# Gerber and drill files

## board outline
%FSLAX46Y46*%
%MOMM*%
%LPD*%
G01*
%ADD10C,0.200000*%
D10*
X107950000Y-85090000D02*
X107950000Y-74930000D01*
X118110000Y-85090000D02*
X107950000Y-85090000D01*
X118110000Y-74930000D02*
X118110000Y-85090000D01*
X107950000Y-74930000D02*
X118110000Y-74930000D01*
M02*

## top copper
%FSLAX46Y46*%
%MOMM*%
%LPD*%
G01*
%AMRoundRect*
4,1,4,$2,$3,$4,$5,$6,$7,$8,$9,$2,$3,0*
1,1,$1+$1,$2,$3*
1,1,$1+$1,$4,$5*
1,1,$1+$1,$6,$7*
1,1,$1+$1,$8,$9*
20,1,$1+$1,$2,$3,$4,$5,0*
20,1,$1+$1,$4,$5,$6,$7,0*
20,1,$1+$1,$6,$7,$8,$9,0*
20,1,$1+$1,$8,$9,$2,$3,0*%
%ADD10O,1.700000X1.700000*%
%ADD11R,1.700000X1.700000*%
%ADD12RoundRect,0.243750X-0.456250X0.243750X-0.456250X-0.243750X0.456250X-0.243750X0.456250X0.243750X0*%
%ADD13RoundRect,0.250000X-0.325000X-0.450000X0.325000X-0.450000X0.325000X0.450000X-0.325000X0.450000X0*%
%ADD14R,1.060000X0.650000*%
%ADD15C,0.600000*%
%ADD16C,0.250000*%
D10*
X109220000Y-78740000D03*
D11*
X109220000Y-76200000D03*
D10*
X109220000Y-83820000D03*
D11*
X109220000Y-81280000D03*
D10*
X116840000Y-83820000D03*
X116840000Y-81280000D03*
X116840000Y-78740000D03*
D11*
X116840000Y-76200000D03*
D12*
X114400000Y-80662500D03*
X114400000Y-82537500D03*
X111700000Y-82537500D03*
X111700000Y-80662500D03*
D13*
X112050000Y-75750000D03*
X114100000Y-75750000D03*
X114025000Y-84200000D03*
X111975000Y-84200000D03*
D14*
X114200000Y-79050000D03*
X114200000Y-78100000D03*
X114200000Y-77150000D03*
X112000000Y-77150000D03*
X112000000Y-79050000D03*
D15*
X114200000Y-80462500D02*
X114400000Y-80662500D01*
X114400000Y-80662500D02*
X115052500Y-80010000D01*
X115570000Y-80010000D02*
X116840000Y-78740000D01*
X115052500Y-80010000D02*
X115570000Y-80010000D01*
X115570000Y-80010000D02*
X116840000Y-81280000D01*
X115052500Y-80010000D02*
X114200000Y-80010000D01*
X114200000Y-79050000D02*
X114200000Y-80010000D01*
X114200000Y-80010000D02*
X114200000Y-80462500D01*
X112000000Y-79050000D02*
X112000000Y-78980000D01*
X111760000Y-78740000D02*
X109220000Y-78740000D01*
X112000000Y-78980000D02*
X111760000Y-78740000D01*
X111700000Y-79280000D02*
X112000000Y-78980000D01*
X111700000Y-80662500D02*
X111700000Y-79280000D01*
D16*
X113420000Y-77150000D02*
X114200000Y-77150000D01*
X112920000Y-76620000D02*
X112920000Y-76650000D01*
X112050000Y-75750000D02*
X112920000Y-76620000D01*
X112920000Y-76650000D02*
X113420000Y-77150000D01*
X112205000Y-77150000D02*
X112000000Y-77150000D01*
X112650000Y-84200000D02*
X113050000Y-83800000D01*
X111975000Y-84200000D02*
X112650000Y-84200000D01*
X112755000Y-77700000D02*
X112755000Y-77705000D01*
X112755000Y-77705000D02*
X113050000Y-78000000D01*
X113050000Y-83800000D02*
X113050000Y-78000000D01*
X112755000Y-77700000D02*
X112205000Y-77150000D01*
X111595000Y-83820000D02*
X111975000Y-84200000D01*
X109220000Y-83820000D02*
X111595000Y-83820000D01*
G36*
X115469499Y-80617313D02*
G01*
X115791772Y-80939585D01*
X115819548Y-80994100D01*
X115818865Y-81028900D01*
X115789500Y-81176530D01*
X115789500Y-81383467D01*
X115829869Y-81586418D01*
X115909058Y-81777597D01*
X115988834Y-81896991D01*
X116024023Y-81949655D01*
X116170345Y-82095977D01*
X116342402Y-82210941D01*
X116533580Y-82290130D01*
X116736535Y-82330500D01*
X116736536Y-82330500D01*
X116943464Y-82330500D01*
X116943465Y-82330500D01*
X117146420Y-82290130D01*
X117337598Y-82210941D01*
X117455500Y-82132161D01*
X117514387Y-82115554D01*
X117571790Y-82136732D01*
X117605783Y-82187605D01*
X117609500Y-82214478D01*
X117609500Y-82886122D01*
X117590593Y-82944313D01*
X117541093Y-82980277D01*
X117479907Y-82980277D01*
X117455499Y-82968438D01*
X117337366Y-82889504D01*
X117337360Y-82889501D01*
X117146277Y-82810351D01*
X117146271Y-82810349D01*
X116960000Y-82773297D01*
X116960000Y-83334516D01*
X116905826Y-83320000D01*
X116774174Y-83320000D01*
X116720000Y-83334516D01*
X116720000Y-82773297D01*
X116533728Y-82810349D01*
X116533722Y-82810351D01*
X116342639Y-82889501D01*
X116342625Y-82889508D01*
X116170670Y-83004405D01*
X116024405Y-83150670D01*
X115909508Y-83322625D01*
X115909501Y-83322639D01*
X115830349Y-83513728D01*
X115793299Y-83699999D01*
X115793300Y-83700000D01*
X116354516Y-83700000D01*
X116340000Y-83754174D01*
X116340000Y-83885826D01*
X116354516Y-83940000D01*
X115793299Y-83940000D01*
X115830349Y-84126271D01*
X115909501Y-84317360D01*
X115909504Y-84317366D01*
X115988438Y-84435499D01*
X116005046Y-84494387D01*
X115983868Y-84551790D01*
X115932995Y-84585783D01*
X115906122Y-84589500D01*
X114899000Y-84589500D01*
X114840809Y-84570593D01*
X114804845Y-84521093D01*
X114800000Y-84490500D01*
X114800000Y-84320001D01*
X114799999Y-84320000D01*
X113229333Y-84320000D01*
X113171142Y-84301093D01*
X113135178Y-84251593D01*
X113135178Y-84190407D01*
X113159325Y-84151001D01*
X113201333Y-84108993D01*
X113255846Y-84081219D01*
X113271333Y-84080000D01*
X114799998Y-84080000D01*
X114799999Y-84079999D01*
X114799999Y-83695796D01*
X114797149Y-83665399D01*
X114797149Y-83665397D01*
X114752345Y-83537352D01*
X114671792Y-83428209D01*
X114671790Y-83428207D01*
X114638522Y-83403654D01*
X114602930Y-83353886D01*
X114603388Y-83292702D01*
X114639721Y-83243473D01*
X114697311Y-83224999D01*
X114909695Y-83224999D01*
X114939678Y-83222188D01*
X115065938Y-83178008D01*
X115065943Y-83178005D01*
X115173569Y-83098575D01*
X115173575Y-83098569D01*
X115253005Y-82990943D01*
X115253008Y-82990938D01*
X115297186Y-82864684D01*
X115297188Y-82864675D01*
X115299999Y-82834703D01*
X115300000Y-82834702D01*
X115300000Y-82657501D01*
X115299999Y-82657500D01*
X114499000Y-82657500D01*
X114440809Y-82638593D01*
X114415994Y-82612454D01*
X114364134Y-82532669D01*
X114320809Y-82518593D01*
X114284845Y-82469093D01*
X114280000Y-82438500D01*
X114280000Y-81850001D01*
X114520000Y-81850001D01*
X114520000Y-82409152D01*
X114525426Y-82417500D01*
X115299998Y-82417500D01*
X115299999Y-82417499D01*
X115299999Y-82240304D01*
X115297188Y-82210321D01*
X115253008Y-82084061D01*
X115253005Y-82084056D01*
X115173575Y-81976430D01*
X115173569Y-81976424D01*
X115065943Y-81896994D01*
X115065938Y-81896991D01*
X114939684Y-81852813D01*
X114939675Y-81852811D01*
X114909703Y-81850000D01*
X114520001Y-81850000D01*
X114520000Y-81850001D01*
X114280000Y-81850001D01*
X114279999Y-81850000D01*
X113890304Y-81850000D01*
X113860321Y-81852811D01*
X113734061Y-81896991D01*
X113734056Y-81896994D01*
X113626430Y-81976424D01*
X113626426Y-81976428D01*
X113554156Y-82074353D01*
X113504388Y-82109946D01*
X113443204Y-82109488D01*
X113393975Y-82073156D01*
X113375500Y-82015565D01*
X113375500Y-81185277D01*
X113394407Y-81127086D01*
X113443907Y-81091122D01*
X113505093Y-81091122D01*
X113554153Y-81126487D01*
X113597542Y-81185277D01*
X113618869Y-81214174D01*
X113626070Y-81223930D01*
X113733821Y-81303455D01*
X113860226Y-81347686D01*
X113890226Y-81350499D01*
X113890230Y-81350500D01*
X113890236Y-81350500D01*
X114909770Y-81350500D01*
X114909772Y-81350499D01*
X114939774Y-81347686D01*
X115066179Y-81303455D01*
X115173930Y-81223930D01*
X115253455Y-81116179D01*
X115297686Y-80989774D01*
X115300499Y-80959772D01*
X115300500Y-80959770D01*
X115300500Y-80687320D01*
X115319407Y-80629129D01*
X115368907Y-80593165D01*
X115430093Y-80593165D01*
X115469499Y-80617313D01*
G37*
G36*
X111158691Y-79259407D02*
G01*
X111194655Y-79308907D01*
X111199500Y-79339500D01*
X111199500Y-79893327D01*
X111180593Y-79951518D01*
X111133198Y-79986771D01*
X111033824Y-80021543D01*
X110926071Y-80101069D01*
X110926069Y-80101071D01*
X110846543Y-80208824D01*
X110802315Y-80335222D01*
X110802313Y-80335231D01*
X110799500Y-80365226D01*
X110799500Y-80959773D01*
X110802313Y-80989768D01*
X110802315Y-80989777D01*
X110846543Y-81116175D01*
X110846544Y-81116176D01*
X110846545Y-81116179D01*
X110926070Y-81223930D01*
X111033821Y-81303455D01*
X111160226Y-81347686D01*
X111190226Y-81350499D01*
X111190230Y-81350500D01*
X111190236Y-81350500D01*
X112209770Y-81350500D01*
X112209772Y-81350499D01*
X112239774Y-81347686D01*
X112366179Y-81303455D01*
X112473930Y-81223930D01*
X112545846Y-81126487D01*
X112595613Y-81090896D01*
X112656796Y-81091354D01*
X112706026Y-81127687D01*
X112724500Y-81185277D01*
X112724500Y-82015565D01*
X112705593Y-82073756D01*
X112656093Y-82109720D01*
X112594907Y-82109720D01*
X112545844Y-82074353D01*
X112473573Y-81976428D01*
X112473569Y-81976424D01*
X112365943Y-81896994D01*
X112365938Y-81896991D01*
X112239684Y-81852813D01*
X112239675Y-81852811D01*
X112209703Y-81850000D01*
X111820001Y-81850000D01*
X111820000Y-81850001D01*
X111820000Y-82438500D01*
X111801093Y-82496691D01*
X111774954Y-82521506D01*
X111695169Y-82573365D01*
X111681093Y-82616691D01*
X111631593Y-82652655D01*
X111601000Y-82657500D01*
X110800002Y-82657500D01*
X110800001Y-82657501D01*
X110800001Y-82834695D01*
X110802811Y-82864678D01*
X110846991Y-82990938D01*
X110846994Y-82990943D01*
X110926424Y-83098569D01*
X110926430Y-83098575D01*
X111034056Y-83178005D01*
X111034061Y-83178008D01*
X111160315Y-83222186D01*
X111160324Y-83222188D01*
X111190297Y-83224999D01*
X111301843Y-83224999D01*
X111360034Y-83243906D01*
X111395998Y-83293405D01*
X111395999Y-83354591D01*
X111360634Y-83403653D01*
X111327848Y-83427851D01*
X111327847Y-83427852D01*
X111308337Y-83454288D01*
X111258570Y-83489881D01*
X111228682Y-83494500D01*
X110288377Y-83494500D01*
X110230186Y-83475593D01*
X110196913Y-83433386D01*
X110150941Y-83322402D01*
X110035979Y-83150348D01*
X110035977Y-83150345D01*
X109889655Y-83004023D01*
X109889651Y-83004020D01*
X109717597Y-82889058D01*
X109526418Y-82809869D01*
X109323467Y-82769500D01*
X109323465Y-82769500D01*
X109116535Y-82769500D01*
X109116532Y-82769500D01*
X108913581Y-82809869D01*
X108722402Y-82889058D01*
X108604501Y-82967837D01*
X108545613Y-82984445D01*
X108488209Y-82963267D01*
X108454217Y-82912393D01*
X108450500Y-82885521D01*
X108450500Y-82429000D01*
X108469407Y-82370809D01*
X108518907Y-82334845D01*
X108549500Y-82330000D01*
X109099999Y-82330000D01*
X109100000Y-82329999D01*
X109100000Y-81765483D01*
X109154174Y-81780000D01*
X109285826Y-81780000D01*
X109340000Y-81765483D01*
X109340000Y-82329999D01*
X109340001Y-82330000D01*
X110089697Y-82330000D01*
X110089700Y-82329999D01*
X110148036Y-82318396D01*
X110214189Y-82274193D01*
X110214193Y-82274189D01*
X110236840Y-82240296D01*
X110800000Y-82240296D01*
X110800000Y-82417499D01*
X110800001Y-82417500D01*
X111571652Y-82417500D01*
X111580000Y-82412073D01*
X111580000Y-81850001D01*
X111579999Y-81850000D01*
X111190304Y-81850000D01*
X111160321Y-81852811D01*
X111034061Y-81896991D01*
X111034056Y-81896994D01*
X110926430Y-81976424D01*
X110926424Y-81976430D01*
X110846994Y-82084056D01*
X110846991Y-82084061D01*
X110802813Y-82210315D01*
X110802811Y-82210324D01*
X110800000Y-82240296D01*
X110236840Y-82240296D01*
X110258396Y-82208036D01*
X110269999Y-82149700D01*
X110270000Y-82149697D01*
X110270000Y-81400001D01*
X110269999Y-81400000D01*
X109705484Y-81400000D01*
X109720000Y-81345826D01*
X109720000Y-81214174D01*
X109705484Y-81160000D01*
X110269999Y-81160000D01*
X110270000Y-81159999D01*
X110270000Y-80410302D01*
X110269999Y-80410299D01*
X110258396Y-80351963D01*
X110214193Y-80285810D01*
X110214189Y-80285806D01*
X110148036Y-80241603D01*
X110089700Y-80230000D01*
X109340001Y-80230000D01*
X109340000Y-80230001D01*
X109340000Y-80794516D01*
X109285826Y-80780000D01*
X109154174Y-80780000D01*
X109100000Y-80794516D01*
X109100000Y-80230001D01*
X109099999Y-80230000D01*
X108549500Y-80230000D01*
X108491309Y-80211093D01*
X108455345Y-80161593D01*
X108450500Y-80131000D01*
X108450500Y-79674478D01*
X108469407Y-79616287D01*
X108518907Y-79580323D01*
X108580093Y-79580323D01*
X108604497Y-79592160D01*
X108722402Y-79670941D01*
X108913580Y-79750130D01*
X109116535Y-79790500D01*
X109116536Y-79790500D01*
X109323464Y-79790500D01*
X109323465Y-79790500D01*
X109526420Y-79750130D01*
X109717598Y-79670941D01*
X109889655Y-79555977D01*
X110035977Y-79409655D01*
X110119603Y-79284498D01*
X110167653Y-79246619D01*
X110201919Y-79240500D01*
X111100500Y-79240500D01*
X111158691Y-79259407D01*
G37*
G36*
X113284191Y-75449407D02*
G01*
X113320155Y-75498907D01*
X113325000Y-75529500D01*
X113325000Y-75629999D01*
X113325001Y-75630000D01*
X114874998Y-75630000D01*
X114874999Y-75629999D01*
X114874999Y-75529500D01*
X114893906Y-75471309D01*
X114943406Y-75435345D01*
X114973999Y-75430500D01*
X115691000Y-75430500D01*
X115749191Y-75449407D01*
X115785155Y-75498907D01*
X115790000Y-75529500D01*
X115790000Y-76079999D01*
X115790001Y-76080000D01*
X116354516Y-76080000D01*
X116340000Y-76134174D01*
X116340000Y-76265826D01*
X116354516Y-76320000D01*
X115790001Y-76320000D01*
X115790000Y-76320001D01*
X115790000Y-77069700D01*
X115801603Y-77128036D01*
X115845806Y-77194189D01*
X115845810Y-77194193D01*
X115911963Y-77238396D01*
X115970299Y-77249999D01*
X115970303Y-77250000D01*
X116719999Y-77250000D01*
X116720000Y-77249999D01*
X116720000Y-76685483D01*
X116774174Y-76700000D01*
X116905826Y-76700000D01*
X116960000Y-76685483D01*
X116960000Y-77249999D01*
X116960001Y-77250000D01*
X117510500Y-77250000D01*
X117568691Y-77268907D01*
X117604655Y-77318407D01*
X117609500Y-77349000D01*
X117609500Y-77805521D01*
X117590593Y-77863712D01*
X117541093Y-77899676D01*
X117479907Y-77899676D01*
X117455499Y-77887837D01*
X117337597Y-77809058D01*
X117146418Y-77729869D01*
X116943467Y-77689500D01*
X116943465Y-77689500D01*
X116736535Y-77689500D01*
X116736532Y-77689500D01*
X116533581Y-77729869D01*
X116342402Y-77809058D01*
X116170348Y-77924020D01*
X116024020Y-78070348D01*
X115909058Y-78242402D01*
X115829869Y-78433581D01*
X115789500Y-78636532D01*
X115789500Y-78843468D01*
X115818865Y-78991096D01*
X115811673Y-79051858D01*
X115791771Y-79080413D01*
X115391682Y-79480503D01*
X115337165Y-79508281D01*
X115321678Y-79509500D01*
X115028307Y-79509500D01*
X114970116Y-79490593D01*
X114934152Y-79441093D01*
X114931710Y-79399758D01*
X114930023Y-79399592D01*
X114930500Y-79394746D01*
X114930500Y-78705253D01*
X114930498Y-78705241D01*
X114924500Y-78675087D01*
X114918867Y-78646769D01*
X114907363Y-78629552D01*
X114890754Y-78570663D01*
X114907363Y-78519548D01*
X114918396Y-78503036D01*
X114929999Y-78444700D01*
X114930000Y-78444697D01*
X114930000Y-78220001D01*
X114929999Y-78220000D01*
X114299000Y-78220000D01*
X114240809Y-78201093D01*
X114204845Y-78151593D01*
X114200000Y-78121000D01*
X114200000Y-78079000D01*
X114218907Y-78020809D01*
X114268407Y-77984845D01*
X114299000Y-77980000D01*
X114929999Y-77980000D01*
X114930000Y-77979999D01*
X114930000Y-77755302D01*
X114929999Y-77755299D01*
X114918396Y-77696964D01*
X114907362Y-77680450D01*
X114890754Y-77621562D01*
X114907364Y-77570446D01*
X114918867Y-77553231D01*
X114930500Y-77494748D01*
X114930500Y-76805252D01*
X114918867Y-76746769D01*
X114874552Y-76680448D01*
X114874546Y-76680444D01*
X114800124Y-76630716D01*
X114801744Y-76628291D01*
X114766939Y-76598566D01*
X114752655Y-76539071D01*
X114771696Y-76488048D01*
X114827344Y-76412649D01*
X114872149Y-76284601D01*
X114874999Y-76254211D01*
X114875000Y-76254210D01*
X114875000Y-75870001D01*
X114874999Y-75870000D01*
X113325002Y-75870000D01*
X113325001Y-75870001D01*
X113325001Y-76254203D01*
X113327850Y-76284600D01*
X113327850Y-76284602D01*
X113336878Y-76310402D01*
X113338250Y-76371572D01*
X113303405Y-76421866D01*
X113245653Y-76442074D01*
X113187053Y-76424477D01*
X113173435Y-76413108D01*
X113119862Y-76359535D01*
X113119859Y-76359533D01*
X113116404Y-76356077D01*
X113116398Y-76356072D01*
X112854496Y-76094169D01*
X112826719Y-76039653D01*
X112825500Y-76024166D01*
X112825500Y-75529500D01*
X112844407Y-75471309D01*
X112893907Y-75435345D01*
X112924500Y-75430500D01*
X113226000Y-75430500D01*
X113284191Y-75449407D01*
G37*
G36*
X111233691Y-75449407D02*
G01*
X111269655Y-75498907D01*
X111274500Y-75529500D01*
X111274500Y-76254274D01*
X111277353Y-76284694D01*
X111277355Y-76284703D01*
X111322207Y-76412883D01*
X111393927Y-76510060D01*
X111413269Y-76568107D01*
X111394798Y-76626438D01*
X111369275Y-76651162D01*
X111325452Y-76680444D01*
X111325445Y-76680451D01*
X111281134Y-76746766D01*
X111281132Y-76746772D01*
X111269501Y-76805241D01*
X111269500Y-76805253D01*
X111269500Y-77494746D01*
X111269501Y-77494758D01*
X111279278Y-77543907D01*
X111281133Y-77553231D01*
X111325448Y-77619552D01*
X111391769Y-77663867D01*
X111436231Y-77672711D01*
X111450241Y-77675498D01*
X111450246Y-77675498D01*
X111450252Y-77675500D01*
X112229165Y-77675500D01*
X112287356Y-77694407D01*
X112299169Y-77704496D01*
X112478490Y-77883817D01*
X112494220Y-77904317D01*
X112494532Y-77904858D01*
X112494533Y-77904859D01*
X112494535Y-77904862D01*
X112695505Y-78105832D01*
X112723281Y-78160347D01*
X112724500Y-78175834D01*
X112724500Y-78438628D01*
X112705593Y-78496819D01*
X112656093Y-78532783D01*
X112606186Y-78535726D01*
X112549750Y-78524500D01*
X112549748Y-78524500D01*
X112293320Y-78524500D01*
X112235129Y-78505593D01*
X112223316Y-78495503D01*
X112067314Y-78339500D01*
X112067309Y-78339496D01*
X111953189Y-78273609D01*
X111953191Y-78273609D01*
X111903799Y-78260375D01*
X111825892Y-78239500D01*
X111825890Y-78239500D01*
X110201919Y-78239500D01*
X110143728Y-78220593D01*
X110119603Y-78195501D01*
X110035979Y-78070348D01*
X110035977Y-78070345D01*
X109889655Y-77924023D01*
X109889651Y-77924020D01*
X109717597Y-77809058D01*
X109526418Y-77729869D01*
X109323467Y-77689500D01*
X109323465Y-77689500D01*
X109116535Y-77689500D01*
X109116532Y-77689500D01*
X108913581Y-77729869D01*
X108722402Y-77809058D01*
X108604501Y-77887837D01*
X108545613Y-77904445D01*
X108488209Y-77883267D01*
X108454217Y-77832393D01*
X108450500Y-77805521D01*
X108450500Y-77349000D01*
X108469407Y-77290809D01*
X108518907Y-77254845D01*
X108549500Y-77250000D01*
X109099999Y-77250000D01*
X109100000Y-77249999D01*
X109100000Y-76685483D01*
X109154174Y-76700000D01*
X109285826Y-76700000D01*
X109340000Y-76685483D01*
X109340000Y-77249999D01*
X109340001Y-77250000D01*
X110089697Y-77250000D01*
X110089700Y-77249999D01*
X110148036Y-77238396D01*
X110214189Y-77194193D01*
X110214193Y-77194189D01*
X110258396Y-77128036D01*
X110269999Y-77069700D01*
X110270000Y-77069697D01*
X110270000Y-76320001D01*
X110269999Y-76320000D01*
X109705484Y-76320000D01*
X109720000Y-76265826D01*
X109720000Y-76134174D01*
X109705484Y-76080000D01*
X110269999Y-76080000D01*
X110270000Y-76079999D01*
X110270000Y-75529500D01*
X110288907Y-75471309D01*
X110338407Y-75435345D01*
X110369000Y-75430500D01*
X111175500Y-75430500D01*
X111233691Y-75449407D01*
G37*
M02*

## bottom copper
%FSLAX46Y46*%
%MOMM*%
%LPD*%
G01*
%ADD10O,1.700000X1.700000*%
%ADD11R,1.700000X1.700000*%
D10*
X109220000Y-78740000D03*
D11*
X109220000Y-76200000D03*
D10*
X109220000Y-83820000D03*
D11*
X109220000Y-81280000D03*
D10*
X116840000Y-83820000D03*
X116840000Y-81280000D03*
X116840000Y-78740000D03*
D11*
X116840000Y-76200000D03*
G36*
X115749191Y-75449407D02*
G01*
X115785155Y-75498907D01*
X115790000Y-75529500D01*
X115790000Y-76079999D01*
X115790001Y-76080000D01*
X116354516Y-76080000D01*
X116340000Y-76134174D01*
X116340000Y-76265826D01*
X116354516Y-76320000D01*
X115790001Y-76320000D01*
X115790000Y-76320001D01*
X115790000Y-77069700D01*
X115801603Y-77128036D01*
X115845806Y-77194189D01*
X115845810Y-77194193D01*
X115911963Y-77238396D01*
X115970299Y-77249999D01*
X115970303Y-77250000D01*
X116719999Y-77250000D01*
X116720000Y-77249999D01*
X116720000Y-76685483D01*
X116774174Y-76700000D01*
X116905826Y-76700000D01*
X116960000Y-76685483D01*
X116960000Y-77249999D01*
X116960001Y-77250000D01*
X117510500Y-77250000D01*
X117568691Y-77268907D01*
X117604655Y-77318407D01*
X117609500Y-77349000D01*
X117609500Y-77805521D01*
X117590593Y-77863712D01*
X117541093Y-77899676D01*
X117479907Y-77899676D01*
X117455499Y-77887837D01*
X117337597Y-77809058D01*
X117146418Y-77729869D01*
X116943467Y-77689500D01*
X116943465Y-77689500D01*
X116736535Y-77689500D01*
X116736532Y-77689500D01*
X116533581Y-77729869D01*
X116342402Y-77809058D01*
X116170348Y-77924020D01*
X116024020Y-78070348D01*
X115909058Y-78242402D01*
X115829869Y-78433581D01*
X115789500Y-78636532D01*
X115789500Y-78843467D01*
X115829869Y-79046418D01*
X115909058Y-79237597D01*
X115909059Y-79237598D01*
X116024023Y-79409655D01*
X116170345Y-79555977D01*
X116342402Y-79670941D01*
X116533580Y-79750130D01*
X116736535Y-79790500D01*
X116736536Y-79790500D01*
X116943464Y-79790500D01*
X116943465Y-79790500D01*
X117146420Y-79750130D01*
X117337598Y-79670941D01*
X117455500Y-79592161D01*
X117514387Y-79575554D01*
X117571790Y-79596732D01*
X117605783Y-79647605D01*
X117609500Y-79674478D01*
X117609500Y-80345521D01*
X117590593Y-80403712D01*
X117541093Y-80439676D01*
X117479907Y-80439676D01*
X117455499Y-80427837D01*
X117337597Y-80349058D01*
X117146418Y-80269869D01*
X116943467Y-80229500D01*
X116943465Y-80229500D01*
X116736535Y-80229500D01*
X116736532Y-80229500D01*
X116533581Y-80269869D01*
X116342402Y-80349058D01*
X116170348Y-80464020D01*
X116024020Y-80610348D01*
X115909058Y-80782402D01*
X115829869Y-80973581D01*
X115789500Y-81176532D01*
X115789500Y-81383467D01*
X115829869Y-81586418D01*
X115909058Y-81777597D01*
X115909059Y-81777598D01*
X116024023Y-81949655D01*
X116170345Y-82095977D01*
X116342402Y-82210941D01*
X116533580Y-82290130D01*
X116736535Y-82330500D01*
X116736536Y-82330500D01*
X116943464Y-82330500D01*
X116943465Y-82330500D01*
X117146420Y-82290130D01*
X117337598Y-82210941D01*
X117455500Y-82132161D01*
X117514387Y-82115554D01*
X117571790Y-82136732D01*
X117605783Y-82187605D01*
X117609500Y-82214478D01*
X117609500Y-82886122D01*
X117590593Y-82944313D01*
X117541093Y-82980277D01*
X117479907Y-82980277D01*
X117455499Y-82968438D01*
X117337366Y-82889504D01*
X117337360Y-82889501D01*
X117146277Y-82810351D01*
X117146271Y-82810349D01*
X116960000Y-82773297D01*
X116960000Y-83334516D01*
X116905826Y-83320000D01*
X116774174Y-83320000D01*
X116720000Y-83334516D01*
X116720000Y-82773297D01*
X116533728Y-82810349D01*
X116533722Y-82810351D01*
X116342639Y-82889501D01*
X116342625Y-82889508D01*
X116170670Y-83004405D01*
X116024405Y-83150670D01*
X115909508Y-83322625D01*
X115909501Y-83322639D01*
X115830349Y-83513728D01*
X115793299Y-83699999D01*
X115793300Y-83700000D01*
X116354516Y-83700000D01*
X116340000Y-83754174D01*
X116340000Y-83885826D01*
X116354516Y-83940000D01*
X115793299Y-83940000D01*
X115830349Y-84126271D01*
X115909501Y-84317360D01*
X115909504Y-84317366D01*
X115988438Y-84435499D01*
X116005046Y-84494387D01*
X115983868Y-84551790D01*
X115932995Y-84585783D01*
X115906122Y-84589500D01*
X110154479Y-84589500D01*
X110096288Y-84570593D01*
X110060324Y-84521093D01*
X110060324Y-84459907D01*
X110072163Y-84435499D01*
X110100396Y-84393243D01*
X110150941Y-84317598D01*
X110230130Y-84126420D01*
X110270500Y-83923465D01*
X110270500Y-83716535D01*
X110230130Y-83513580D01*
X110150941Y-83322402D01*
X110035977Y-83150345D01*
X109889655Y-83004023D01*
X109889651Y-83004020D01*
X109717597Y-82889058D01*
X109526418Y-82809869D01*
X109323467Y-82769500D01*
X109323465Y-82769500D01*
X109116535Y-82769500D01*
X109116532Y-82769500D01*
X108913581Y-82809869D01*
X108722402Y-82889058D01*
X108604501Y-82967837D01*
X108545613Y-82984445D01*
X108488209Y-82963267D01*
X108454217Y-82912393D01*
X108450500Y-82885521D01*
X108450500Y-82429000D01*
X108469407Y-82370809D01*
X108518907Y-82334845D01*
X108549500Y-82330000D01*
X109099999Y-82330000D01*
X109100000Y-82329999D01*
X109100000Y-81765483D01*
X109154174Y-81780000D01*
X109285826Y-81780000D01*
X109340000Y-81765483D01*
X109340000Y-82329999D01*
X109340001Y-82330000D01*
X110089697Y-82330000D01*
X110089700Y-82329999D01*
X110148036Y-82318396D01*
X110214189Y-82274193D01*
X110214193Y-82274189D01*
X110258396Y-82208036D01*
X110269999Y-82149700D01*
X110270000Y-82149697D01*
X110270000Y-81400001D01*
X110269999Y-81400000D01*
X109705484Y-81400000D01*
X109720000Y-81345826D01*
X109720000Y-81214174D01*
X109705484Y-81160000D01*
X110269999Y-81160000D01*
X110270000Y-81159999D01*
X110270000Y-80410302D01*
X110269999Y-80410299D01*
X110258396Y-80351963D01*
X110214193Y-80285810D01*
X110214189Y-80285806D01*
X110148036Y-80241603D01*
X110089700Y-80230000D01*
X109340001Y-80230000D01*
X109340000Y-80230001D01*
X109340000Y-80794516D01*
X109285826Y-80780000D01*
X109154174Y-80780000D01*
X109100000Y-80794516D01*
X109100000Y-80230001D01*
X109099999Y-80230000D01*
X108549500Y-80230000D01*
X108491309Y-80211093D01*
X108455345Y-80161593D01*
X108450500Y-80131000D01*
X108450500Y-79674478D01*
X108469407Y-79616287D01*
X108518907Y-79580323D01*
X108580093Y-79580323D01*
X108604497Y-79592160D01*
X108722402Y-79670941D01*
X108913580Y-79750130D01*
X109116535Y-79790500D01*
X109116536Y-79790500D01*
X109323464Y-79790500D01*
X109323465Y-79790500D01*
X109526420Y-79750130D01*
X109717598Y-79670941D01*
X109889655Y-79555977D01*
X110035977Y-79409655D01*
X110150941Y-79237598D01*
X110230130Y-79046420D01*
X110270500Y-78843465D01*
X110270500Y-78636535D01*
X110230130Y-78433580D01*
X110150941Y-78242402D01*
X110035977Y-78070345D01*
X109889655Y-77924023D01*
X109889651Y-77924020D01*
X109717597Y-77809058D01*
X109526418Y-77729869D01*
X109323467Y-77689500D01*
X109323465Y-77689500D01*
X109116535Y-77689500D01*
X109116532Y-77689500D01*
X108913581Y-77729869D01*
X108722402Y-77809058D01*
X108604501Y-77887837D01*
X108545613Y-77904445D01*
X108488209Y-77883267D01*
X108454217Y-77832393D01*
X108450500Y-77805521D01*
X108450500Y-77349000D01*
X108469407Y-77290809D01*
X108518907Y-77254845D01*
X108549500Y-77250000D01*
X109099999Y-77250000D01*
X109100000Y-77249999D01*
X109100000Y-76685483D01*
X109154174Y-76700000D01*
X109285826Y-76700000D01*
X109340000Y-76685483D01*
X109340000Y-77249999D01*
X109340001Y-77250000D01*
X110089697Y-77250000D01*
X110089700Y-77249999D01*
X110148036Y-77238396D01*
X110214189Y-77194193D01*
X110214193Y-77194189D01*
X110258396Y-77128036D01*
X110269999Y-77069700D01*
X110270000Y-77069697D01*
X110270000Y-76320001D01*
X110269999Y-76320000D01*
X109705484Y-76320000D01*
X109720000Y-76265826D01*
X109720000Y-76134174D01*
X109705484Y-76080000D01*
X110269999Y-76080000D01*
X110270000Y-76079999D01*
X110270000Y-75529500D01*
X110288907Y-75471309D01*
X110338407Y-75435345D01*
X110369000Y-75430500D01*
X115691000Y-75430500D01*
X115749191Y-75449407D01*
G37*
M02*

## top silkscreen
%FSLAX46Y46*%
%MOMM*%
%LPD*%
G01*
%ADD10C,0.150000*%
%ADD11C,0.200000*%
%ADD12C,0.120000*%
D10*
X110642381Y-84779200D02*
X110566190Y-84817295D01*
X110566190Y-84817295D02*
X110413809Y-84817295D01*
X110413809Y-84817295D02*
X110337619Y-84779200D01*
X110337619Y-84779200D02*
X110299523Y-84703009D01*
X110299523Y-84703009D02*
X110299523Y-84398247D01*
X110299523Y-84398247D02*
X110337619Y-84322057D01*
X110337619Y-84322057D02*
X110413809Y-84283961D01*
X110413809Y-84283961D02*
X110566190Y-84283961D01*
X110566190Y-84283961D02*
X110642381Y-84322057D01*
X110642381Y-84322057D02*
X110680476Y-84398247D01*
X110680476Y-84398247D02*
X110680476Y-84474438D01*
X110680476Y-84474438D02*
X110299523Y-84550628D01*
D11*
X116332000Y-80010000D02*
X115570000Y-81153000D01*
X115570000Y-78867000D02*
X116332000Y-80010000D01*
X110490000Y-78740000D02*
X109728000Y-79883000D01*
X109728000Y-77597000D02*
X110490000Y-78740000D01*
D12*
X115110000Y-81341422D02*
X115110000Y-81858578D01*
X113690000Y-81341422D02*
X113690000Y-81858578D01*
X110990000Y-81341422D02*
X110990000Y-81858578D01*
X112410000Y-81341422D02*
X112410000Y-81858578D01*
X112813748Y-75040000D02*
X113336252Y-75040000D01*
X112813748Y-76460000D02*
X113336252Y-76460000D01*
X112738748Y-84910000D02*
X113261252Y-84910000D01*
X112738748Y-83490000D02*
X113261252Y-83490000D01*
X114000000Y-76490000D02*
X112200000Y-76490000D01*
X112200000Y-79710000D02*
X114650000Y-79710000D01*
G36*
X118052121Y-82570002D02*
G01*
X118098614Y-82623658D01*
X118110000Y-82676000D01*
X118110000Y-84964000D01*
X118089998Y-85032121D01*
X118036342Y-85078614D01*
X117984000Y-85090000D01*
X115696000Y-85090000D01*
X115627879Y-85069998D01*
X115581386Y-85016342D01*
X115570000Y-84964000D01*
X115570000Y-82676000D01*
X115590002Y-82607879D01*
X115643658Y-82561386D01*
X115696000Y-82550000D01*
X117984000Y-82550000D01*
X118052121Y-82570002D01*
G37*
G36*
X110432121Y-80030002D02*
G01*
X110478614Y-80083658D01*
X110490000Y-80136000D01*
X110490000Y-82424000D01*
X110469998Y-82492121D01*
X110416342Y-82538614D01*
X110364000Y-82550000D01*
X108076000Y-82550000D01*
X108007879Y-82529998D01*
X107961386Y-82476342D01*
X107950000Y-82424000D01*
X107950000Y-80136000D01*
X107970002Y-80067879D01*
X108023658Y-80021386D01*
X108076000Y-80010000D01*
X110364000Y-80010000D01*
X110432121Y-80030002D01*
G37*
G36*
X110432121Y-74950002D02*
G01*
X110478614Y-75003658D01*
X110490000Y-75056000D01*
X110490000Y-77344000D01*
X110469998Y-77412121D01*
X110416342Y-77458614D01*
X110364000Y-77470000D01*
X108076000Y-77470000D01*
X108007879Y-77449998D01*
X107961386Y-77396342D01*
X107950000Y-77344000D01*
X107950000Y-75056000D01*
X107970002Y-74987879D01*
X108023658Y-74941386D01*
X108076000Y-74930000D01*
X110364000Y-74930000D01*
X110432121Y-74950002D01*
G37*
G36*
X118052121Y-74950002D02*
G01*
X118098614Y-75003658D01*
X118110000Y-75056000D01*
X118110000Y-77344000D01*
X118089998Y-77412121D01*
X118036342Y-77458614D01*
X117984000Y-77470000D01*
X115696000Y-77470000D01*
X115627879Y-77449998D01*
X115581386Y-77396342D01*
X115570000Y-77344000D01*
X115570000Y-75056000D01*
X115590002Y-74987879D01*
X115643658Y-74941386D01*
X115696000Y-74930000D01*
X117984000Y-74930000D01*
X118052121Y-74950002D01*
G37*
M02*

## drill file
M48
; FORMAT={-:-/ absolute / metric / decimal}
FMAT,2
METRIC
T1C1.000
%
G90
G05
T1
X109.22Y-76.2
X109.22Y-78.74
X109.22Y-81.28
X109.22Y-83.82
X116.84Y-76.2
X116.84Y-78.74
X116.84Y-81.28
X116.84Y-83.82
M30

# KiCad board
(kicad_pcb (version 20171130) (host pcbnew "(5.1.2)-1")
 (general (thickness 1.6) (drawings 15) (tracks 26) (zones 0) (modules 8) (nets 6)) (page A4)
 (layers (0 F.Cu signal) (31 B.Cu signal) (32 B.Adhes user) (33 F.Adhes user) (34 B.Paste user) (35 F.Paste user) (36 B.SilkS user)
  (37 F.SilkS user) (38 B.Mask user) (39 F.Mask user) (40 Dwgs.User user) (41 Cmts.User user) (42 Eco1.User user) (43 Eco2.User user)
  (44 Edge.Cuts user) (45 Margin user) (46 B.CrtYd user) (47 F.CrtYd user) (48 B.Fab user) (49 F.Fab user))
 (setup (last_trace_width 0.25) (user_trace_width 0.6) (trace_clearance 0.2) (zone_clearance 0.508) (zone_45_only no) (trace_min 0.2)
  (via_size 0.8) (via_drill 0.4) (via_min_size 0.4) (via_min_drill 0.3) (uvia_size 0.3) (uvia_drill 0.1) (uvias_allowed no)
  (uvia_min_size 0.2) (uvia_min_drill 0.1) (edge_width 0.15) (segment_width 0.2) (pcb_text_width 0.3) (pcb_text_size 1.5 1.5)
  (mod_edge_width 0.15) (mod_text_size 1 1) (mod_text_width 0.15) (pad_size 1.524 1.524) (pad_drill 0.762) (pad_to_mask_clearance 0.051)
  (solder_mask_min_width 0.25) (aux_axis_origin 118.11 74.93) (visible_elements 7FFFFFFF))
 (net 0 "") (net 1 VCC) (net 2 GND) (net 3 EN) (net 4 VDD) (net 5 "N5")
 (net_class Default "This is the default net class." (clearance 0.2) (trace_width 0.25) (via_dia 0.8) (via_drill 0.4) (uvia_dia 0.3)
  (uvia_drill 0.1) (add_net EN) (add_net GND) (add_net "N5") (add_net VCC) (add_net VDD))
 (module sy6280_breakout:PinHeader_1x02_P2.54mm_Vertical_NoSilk (layer F.Cu) (at 109.22 76.2)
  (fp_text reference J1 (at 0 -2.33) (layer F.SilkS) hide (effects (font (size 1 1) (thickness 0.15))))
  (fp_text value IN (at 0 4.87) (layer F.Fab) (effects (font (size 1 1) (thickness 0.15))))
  (pad 2 thru_hole oval (at 0 2.54) (size 1.7 1.7) (drill 1) (layers *.Cu *.Mask) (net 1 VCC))
  (pad 1 thru_hole rect (at 0 0) (size 1.7 1.7) (drill 1) (layers *.Cu *.Mask) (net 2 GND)))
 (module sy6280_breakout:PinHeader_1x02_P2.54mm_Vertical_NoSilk (layer F.Cu) (at 109.22 81.28)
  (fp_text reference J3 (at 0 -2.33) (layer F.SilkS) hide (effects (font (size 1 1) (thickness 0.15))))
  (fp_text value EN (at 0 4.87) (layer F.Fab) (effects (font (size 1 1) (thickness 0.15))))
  (pad 2 thru_hole oval (at 0 2.54) (size 1.7 1.7) (drill 1) (layers *.Cu *.Mask) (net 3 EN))
  (pad 1 thru_hole rect (at 0 0) (size 1.7 1.7) (drill 1) (layers *.Cu *.Mask) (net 2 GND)))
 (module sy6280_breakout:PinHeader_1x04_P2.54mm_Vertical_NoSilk (layer F.Cu) (at 116.84 76.2)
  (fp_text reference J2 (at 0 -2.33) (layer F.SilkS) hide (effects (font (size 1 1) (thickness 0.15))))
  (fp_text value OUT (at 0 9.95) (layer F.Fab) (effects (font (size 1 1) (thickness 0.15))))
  (pad 4 thru_hole oval (at 0 7.62) (size 1.7 1.7) (drill 1) (layers *.Cu *.Mask) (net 2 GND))
  (pad 3 thru_hole oval (at 0 5.08) (size 1.7 1.7) (drill 1) (layers *.Cu *.Mask) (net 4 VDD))
  (pad 2 thru_hole oval (at 0 2.54) (size 1.7 1.7) (drill 1) (layers *.Cu *.Mask) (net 4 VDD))
  (pad 1 thru_hole rect (at 0 0) (size 1.7 1.7) (drill 1) (layers *.Cu *.Mask) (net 2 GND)))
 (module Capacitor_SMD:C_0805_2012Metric (layer F.Cu) (at 114.4 81.6 270)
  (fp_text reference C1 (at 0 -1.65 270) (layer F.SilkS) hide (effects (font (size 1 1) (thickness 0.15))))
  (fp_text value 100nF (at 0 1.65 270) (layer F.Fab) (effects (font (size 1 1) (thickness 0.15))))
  (fp_line (start -0.258578 -0.71) (end 0.258578 -0.71) (layer F.SilkS) (width 0.12))
  (fp_line (start -0.258578 0.71) (end 0.258578 0.71) (layer F.SilkS) (width 0.12))
  (pad 1 smd roundrect (at -0.9375 0 270) (size 0.975 1.4) (layers F.Cu F.Paste F.Mask) (roundrect_rratio 0.25) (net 4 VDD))
  (pad 2 smd roundrect (at 0.9375 0 270) (size 0.975 1.4) (layers F.Cu F.Paste F.Mask) (roundrect_rratio 0.25) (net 2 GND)))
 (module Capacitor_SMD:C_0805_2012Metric (layer F.Cu) (at 111.7 81.6 270)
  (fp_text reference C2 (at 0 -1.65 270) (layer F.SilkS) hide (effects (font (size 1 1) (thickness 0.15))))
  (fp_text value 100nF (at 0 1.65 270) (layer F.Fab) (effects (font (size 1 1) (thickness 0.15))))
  (fp_line (start -0.258578 0.71) (end 0.258578 0.71) (layer F.SilkS) (width 0.12))
  (fp_line (start -0.258578 -0.71) (end 0.258578 -0.71) (layer F.SilkS) (width 0.12))
  (pad 2 smd roundrect (at 0.9375 0 270) (size 0.975 1.4) (layers F.Cu F.Paste F.Mask) (roundrect_rratio 0.25) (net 2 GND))
  (pad 1 smd roundrect (at -0.9375 0 270) (size 0.975 1.4) (layers F.Cu F.Paste F.Mask) (roundrect_rratio 0.25) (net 1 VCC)))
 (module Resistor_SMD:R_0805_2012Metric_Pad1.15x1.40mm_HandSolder (layer F.Cu) (at 113.075 75.75)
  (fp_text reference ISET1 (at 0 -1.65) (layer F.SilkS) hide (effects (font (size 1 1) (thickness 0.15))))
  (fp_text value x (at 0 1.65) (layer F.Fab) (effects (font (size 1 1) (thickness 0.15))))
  (fp_line (start -0.261252 -0.71) (end 0.261252 -0.71) (layer F.SilkS) (width 0.12))
  (fp_line (start -0.261252 0.71) (end 0.261252 0.71) (layer F.SilkS) (width 0.12))
  (pad 1 smd roundrect (at -1.025 0) (size 1.15 1.4) (layers F.Cu F.Paste F.Mask) (roundrect_rratio 0.217391) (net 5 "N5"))
  (pad 2 smd roundrect (at 1.025 0) (size 1.15 1.4) (layers F.Cu F.Paste F.Mask) (roundrect_rratio 0.217391) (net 2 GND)))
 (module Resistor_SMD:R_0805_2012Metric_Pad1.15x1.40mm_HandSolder (layer F.Cu) (at 113 84.2)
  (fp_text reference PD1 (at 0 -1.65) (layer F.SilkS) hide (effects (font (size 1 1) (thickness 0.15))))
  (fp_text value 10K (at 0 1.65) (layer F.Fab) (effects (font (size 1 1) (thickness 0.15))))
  (fp_line (start -0.261252 0.71) (end 0.261252 0.71) (layer F.SilkS) (width 0.12))
  (fp_line (start -0.261252 -0.71) (end 0.261252 -0.71) (layer F.SilkS) (width 0.12))
  (pad 2 smd roundrect (at 1.025 0) (size 1.15 1.4) (layers F.Cu F.Paste F.Mask) (roundrect_rratio 0.217391) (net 2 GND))
  (pad 1 smd roundrect (at -1.025 0) (size 1.15 1.4) (layers F.Cu F.Paste F.Mask) (roundrect_rratio 0.217391) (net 3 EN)))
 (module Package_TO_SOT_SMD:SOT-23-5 (layer F.Cu) (at 113.1 78.1 180)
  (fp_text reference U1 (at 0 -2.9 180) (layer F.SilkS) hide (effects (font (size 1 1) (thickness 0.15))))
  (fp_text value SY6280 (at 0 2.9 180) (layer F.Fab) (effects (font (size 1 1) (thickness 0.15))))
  (fp_line (start -0.9 1.61) (end 0.9 1.61) (layer F.SilkS) (width 0.12))
  (fp_line (start 0.9 -1.61) (end -1.55 -1.61) (layer F.SilkS) (width 0.12))
  (pad 1 smd rect (at -1.1 -0.95 180) (size 1.06 0.65) (layers F.Cu F.Paste F.Mask) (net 4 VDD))
  (pad 2 smd rect (at -1.1 0 180) (size 1.06 0.65) (layers F.Cu F.Paste F.Mask) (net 2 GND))
  (pad 3 smd rect (at -1.1 0.95 180) (size 1.06 0.65) (layers F.Cu F.Paste F.Mask) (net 5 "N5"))
  (pad 4 smd rect (at 1.1 0.95 180) (size 1.06 0.65) (layers F.Cu F.Paste F.Mask) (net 3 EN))
  (pad 5 smd rect (at 1.1 -0.95 180) (size 1.06 0.65) (layers F.Cu F.Paste F.Mask) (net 1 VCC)))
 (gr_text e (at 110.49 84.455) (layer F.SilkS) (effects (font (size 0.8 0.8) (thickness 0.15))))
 (gr_line (start 116.332 80.01) (end 115.57 81.153) (layer F.SilkS) (width 0.2))
 (gr_line (start 115.57 78.867) (end 116.332 80.01) (layer F.SilkS) (width 0.2))
 (gr_line (start 110.49 78.74) (end 109.728 79.883) (layer F.SilkS) (width 0.2))
 (gr_line (start 109.728 77.597) (end 110.49 78.74) (layer F.SilkS) (width 0.2))
 (gr_line (start 107.95 85.09) (end 107.95 74.93) (layer Edge.Cuts) (width 0.2))
 (gr_line (start 118.11 85.09) (end 107.95 85.09) (layer Edge.Cuts) (width 0.2))
 (gr_line (start 118.11 74.93) (end 118.11 85.09) (layer Edge.Cuts) (width 0.2))
 (gr_line (start 107.95 74.93) (end 118.11 74.93) (layer Edge.Cuts) (width 0.2))
 (segment (start 114.2 80.4625) (end 114.4 80.6625) (width 0.6) (layer F.Cu) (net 4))
 (segment (start 114.4 80.6625) (end 115.0525 80.01) (width 0.6) (layer F.Cu) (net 4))
 (segment (start 115.57 80.01) (end 116.84 78.74) (width 0.6) (layer F.Cu) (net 4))
 (segment (start 115.0525 80.01) (end 115.57 80.01) (width 0.6) (layer F.Cu) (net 4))
 (segment (start 115.57 80.01) (end 116.84 81.28) (width 0.6) (layer F.Cu) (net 4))
 (segment (start 115.0525 80.01) (end 114.2 80.01) (width 0.6) (layer F.Cu) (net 4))
 (segment (start 114.2 79.05) (end 114.2 80.01) (width 0.6) (layer F.Cu) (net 4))
 (segment (start 114.2 80.01) (end 114.2 80.4625) (width 0.6) (layer F.Cu) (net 4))
 (segment (start 112 79.05) (end 112 78.98) (width 0.6) (layer F.Cu) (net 1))
 (segment (start 111.76 78.74) (end 109.22 78.74) (width 0.6) (layer F.Cu) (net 1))
 (segment (start 112 78.98) (end 111.76 78.74) (width 0.6) (layer F.Cu) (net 1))
 (segment (start 111.7 79.28) (end 112 78.98) (width 0.6) (layer F.Cu) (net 1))
 (segment (start 111.7 80.6625) (end 111.7 79.28) (width 0.6) (layer F.Cu) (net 1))
 (segment (start 113.42 77.15) (end 114.2 77.15) (width 0.25) (layer F.Cu) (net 5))
 (segment (start 112.92 76.62) (end 112.92 76.65) (width 0.25) (layer F.Cu) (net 5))
 (segment (start 112.05 75.75) (end 112.92 76.62) (width 0.25) (layer F.Cu) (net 5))
 (segment (start 112.92 76.65) (end 113.42 77.15) (width 0.25) (layer F.Cu) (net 5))
 (segment (start 112.205 77.15) (end 112 77.15) (width 0.25) (layer F.Cu) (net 3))
 (segment (start 112.65 84.2) (end 113.05 83.8) (width 0.25) (layer F.Cu) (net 3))
 (segment (start 111.975 84.2) (end 112.65 84.2) (width 0.25) (layer F.Cu) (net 3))
 (segment (start 112.755 77.7) (end 112.755 77.705) (width 0.25) (layer F.Cu) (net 3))
 (segment (start 112.755 77.705) (end 113.05 78) (width 0.25) (layer F.Cu) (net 3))
 (segment (start 113.05 83.8) (end 113.05 78) (width 0.25) (layer F.Cu) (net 3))
 (segment (start 112.755 77.7) (end 112.205 77.15) (width 0.25) (layer F.Cu) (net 3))
 (segment (start 111.595 83.82) (end 111.975 84.2) (width 0.25) (layer F.Cu) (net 3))
 (segment (start 109.22 83.82) (end 111.595 83.82) (width 0.25) (layer F.Cu) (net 3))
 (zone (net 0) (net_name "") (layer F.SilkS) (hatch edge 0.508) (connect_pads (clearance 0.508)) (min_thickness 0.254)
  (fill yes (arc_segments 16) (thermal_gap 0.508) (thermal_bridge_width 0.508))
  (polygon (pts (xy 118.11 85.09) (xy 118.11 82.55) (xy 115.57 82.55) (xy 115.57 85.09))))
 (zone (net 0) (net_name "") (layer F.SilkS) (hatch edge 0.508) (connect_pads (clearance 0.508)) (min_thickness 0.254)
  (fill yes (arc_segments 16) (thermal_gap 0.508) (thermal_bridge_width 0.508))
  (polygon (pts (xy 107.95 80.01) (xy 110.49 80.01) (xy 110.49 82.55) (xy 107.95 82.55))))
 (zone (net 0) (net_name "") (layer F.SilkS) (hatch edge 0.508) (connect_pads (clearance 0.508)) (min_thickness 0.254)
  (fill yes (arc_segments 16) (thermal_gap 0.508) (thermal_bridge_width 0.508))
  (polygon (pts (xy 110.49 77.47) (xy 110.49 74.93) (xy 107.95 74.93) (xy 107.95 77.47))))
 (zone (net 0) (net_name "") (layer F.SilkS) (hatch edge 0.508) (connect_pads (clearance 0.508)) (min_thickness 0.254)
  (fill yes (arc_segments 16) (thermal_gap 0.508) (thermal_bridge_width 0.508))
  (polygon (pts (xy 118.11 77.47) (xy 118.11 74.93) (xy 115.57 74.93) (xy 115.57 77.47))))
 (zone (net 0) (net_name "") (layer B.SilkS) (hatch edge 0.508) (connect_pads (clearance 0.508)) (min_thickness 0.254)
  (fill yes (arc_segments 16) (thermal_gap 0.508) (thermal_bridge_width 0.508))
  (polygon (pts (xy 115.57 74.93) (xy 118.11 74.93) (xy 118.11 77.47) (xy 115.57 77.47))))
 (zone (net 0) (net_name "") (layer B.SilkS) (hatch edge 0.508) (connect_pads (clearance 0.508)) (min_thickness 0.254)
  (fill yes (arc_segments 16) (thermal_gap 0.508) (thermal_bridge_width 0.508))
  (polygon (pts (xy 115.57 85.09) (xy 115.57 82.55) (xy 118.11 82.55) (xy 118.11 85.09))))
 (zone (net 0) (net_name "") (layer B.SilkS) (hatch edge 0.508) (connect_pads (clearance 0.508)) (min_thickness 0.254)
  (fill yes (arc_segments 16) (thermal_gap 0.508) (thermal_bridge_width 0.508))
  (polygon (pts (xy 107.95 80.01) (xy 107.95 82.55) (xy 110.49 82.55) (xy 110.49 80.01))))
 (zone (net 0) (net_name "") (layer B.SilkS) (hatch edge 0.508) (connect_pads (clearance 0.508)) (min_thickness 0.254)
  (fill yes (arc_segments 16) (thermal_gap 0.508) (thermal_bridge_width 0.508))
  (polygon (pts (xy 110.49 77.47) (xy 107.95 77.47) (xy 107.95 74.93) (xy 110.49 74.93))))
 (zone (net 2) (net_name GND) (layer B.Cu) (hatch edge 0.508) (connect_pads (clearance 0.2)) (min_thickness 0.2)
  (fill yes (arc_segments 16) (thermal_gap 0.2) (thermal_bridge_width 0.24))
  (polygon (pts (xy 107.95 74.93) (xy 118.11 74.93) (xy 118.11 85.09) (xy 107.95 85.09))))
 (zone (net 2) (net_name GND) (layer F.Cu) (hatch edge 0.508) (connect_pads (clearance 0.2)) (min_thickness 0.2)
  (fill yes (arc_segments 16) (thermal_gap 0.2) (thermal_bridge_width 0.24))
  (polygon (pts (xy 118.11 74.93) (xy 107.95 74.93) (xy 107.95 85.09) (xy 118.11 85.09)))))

